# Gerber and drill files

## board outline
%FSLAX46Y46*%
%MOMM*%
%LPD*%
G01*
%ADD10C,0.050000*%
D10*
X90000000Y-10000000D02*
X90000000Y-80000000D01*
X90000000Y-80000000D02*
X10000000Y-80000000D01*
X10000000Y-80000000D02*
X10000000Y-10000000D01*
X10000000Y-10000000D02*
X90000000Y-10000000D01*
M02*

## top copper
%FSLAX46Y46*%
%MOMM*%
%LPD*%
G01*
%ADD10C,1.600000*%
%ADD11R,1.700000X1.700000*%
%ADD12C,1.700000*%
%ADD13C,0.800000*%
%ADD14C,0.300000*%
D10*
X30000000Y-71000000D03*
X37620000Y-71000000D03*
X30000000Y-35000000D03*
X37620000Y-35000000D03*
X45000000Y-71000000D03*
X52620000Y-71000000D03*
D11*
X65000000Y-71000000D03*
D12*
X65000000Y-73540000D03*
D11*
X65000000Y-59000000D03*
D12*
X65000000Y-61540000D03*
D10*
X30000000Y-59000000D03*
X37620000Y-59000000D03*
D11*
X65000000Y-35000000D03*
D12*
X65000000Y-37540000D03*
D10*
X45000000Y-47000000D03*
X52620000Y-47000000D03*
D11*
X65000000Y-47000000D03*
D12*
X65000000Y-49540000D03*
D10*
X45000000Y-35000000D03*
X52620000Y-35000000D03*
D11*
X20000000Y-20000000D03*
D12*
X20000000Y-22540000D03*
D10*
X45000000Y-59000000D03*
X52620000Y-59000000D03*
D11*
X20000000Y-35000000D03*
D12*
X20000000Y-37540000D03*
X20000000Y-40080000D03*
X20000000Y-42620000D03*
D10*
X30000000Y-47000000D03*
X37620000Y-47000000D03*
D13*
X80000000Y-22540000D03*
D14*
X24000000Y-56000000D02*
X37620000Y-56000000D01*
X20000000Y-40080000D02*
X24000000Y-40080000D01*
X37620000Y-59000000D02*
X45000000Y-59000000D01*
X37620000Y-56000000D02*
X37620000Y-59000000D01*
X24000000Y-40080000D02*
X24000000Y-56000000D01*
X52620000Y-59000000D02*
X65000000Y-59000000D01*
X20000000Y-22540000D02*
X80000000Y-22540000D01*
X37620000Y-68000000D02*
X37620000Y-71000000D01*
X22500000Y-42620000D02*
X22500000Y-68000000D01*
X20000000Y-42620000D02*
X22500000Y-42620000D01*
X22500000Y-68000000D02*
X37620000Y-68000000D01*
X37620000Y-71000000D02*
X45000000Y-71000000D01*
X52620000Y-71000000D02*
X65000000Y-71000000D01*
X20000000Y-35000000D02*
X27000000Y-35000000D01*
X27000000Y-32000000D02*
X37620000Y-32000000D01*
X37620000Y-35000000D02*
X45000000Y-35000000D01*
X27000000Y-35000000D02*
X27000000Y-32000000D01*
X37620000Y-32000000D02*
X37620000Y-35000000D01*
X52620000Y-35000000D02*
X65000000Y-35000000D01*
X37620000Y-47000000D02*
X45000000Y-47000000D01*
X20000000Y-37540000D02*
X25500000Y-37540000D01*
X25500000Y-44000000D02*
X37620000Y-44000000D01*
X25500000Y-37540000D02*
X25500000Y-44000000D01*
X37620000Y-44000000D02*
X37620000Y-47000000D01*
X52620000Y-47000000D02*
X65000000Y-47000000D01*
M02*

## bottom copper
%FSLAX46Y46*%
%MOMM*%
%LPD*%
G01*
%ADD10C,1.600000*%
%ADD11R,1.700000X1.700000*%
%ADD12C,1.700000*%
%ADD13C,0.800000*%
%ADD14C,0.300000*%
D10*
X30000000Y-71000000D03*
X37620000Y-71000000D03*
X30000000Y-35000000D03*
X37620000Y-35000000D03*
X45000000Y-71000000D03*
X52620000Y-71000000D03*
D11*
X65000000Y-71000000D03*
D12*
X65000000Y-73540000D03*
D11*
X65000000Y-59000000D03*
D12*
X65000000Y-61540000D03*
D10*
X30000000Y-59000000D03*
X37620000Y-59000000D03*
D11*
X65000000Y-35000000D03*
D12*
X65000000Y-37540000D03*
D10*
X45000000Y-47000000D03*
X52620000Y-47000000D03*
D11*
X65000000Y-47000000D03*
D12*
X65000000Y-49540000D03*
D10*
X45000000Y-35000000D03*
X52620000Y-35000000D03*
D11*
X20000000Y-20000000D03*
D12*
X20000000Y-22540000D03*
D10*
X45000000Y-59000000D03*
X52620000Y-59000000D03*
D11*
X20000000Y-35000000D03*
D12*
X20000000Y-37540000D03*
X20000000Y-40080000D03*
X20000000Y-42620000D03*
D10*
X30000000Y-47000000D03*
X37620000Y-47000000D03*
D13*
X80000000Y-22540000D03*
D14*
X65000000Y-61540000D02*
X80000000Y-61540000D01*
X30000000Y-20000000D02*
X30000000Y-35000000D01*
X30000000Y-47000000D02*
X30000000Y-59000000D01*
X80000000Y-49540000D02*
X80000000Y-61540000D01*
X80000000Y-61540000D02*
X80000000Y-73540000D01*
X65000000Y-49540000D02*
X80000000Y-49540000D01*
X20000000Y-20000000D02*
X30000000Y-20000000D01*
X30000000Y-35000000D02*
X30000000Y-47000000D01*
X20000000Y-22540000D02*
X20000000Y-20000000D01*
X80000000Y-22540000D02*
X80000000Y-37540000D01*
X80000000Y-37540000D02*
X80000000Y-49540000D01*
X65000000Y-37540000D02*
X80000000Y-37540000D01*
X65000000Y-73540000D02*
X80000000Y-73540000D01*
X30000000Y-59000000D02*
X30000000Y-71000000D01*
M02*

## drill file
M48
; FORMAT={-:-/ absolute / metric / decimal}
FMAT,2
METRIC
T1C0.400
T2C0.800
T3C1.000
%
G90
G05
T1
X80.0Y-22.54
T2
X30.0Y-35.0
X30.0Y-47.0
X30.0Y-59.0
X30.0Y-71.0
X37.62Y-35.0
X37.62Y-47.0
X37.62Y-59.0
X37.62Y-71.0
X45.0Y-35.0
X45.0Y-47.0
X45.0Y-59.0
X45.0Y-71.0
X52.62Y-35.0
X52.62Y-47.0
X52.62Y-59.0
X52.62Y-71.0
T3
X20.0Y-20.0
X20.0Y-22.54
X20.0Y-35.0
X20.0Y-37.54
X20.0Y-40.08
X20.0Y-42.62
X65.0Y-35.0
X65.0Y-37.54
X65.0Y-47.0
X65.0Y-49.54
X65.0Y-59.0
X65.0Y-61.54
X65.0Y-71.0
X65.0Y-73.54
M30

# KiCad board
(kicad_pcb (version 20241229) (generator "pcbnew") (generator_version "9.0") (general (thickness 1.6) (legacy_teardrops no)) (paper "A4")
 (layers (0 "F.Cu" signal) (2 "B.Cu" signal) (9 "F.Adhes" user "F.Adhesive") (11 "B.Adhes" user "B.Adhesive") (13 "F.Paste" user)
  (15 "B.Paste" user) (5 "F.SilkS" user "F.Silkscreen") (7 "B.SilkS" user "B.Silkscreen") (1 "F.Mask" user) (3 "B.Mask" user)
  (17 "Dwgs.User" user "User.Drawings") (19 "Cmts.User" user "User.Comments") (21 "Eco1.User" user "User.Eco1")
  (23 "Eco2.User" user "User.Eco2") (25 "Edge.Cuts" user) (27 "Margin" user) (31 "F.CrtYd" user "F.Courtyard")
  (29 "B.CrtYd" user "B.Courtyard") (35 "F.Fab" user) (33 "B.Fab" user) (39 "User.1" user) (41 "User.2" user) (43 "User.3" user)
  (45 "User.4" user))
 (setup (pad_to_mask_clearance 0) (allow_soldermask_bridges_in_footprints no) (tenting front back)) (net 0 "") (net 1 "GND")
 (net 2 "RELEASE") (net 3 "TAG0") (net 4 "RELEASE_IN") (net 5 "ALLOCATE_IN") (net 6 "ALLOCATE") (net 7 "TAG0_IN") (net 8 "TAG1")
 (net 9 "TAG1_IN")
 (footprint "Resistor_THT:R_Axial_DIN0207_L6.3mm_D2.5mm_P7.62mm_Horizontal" (layer "F.Cu") (at 30 71)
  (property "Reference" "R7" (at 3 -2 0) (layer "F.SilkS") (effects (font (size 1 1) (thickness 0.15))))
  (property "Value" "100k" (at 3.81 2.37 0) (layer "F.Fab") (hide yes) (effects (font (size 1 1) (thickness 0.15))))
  (pad "1" thru_hole circle (at 0 0) (size 1.6 1.6) (drill 0.8) (layers "*.Cu" "*.Mask") (remove_unused_layers no) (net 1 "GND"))
  (pad "2" thru_hole circle (at 7.62 0) (size 1.6 1.6) (drill 0.8) (layers "*.Cu" "*.Mask") (remove_unused_layers no) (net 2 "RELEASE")))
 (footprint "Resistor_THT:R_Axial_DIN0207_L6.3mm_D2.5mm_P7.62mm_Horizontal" (layer "F.Cu") (at 30 35)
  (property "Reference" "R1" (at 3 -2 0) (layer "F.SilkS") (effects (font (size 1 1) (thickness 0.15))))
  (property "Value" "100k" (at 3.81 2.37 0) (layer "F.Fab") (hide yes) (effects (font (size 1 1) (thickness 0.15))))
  (pad "1" thru_hole circle (at 0 0) (size 1.6 1.6) (drill 0.8) (layers "*.Cu" "*.Mask") (remove_unused_layers no) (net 1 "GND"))
  (pad "2" thru_hole circle (at 7.62 0) (size 1.6 1.6) (drill 0.8) (layers "*.Cu" "*.Mask") (remove_unused_layers no) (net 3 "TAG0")))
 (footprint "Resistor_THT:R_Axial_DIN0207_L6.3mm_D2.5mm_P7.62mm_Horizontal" (layer "F.Cu") (at 45 71)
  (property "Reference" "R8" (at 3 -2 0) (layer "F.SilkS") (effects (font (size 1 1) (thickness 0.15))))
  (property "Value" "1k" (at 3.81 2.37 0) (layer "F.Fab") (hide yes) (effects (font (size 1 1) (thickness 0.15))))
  (pad "1" thru_hole circle (at 0 0) (size 1.6 1.6) (drill 0.8) (layers "*.Cu" "*.Mask") (remove_unused_layers no) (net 2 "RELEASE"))
  (pad "2" thru_hole circle (at 7.62 0) (size 1.6 1.6) (drill 0.8) (layers "*.Cu" "*.Mask") (remove_unused_layers no) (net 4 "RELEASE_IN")))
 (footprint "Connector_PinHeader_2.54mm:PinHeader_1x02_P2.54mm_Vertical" (layer "F.Cu") (at 65 71)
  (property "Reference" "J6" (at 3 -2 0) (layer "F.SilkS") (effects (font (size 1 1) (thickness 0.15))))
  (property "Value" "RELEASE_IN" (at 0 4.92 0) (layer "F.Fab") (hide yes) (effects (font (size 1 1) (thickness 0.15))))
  (pad "1" thru_hole rect (at 0 0) (size 1.7 1.7) (drill 1) (layers "*.Cu" "*.Mask") (remove_unused_layers no) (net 4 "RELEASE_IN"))
  (pad "2" thru_hole circle (at 0 2.54) (size 1.7 1.7) (drill 1) (layers "*.Cu" "*.Mask") (remove_unused_layers no) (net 1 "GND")))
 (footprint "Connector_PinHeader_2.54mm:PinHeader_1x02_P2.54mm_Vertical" (layer "F.Cu") (at 65 59)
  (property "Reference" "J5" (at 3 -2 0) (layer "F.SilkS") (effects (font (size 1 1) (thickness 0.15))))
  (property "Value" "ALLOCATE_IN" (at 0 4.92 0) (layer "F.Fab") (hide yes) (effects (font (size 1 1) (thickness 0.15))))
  (pad "1" thru_hole rect (at 0 0) (size 1.7 1.7) (drill 1) (layers "*.Cu" "*.Mask") (remove_unused_layers no) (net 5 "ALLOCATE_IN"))
  (pad "2" thru_hole circle (at 0 2.54) (size 1.7 1.7) (drill 1) (layers "*.Cu" "*.Mask") (remove_unused_layers no) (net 1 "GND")))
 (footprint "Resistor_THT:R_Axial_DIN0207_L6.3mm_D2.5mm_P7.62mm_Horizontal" (layer "F.Cu") (at 30 59)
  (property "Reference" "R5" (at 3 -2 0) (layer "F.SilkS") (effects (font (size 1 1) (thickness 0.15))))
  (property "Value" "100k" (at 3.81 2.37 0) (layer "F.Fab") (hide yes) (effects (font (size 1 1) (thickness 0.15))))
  (pad "1" thru_hole circle (at 0 0) (size 1.6 1.6) (drill 0.8) (layers "*.Cu" "*.Mask") (remove_unused_layers no) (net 1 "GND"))
  (pad "2" thru_hole circle (at 7.62 0) (size 1.6 1.6) (drill 0.8) (layers "*.Cu" "*.Mask") (remove_unused_layers no) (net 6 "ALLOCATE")))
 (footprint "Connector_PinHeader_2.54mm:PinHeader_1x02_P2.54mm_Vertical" (layer "F.Cu") (at 65 35)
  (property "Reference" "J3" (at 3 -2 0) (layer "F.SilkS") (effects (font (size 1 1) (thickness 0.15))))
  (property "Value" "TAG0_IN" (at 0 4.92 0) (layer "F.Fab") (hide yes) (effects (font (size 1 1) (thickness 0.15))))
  (pad "1" thru_hole rect (at 0 0) (size 1.7 1.7) (drill 1) (layers "*.Cu" "*.Mask") (remove_unused_layers no) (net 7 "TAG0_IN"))
  (pad "2" thru_hole circle (at 0 2.54) (size 1.7 1.7) (drill 1) (layers "*.Cu" "*.Mask") (remove_unused_layers no) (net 1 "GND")))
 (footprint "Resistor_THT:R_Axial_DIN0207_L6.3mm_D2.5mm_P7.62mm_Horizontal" (layer "F.Cu") (at 45 47)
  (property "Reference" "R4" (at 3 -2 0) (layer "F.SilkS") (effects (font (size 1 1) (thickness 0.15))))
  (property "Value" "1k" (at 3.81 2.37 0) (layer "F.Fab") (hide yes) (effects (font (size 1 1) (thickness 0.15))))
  (pad "1" thru_hole circle (at 0 0) (size 1.6 1.6) (drill 0.8) (layers "*.Cu" "*.Mask") (remove_unused_layers no) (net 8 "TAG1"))
  (pad "2" thru_hole circle (at 7.62 0) (size 1.6 1.6) (drill 0.8) (layers "*.Cu" "*.Mask") (remove_unused_layers no) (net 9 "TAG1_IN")))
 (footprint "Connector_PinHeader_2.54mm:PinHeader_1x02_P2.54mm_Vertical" (layer "F.Cu") (at 65 47)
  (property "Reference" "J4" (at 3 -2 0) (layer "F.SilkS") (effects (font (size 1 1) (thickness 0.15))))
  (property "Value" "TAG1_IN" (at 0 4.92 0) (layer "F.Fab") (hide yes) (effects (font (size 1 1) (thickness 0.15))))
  (pad "1" thru_hole rect (at 0 0) (size 1.7 1.7) (drill 1) (layers "*.Cu" "*.Mask") (remove_unused_layers no) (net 9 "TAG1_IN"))
  (pad "2" thru_hole circle (at 0 2.54) (size 1.7 1.7) (drill 1) (layers "*.Cu" "*.Mask") (remove_unused_layers no) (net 1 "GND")))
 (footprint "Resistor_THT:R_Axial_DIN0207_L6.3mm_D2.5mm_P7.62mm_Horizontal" (layer "F.Cu") (at 45 35)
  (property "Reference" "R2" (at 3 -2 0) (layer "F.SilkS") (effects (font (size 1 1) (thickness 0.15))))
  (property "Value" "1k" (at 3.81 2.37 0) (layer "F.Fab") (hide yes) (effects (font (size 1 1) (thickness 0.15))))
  (pad "1" thru_hole circle (at 0 0) (size 1.6 1.6) (drill 0.8) (layers "*.Cu" "*.Mask") (remove_unused_layers no) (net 3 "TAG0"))
  (pad "2" thru_hole circle (at 7.62 0) (size 1.6 1.6) (drill 0.8) (layers "*.Cu" "*.Mask") (remove_unused_layers no) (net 7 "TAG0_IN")))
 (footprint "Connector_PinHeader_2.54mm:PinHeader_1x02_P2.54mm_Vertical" (layer "F.Cu") (at 20 20)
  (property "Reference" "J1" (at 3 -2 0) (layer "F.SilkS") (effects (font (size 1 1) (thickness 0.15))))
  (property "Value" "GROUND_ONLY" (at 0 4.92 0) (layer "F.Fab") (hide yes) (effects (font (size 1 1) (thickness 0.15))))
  (pad "1" thru_hole rect (at 0 0) (size 1.7 1.7) (drill 1) (layers "*.Cu" "*.Mask") (remove_unused_layers no) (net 1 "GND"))
  (pad "2" thru_hole circle (at 0 2.54) (size 1.7 1.7) (drill 1) (layers "*.Cu" "*.Mask") (remove_unused_layers no) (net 1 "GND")))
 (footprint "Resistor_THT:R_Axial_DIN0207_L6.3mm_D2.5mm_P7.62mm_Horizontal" (layer "F.Cu") (at 45 59)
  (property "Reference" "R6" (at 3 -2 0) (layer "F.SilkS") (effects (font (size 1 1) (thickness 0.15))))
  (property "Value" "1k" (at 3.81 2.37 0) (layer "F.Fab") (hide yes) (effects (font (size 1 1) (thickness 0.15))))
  (pad "1" thru_hole circle (at 0 0) (size 1.6 1.6) (drill 0.8) (layers "*.Cu" "*.Mask") (remove_unused_layers no) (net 6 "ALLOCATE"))
  (pad "2" thru_hole circle (at 7.62 0) (size 1.6 1.6) (drill 0.8) (layers "*.Cu" "*.Mask") (remove_unused_layers no) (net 5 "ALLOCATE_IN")))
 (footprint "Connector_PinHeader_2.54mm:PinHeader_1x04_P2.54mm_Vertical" (layer "F.Cu") (at 20 35)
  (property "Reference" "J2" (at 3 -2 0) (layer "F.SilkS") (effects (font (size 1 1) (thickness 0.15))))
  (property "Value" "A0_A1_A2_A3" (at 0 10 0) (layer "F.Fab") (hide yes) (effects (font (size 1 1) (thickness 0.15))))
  (pad "1" thru_hole rect (at 0 0) (size 1.7 1.7) (drill 1) (layers "*.Cu" "*.Mask") (remove_unused_layers no) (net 3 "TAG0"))
  (pad "2" thru_hole circle (at 0 2.54) (size 1.7 1.7) (drill 1) (layers "*.Cu" "*.Mask") (remove_unused_layers no) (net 8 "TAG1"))
  (pad "3" thru_hole circle (at 0 5.08) (size 1.7 1.7) (drill 1) (layers "*.Cu" "*.Mask") (remove_unused_layers no) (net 6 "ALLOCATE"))
  (pad "4" thru_hole circle (at 0 7.62) (size 1.7 1.7) (drill 1) (layers "*.Cu" "*.Mask") (remove_unused_layers no) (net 2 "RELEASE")))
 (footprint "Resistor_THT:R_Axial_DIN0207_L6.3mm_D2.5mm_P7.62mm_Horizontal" (layer "F.Cu") (at 30 47)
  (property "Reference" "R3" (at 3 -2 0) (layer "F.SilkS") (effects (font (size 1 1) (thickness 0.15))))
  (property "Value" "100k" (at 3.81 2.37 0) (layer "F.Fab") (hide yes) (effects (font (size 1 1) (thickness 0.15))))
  (pad "1" thru_hole circle (at 0 0) (size 1.6 1.6) (drill 0.8) (layers "*.Cu" "*.Mask") (remove_unused_layers no) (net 1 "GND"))
  (pad "2" thru_hole circle (at 7.62 0) (size 1.6 1.6) (drill 0.8) (layers "*.Cu" "*.Mask") (remove_unused_layers no) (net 8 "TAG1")))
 (gr_line (start 90 10) (end 90 80) (stroke (width 0.05) (type default)) (layer "Edge.Cuts"))
 (gr_line (start 90 80) (end 10 80) (stroke (width 0.05) (type default)) (layer "Edge.Cuts"))
 (gr_line (start 10 80) (end 10 10) (stroke (width 0.05) (type default)) (layer "Edge.Cuts"))
 (gr_line (start 10 10) (end 90 10) (stroke (width 0.05) (type default)) (layer "Edge.Cuts"))
 (segment (start 24 56) (end 37.62 56) (width 0.3) (layer "F.Cu") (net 6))
 (segment (start 20 40.08) (end 24 40.08) (width 0.3) (layer "F.Cu") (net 6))
 (segment (start 37.62 59) (end 45 59) (width 0.3) (layer "F.Cu") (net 6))
 (segment (start 37.62 56) (end 37.62 59) (width 0.3) (layer "F.Cu") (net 6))
 (segment (start 24 40.08) (end 24 56) (width 0.3) (layer "F.Cu") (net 6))
 (segment (start 52.62 59) (end 65 59) (width 0.3) (layer "F.Cu") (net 5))
 (segment (start 20 22.54) (end 80 22.54) (width 0.3) (layer "F.Cu") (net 1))
 (via (at 80 22.54) (size 0.8) (drill 0.4) (layers "F.Cu" "B.Cu") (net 1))
 (segment (start 65 61.54) (end 80 61.54) (width 0.3) (layer "B.Cu") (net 1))
 (segment (start 30 20) (end 30 35) (width 0.3) (layer "B.Cu") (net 1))
 (segment (start 30 47) (end 30 59) (width 0.3) (layer "B.Cu") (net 1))
 (segment (start 80 49.54) (end 80 61.54) (width 0.3) (layer "B.Cu") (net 1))
 (segment (start 80 61.54) (end 80 73.54) (width 0.3) (layer "B.Cu") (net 1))
 (segment (start 65 49.54) (end 80 49.54) (width 0.3) (layer "B.Cu") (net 1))
 (segment (start 20 20) (end 30 20) (width 0.3) (layer "B.Cu") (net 1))
 (segment (start 30 35) (end 30 47) (width 0.3) (layer "B.Cu") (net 1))
 (segment (start 20 22.54) (end 20 20) (width 0.3) (layer "B.Cu") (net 1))
 (segment (start 80 22.54) (end 80 37.54) (width 0.3) (layer "B.Cu") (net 1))
 (segment (start 80 37.54) (end 80 49.54) (width 0.3) (layer "B.Cu") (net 1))
 (segment (start 65 37.54) (end 80 37.54) (width 0.3) (layer "B.Cu") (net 1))
 (segment (start 65 73.54) (end 80 73.54) (width 0.3) (layer "B.Cu") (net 1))
 (segment (start 30 59) (end 30 71) (width 0.3) (layer "B.Cu") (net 1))
 (segment (start 37.62 68) (end 37.62 71) (width 0.3) (layer "F.Cu") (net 2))
 (segment (start 22.5 42.62) (end 22.5 68) (width 0.3) (layer "F.Cu") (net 2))
 (segment (start 20 42.62) (end 22.5 42.62) (width 0.3) (layer "F.Cu") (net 2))
 (segment (start 22.5 68) (end 37.62 68) (width 0.3) (layer "F.Cu") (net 2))
 (segment (start 37.62 71) (end 45 71) (width 0.3) (layer "F.Cu") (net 2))
 (segment (start 52.62 71) (end 65 71) (width 0.3) (layer "F.Cu") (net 4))
 (segment (start 20 35) (end 27 35) (width 0.3) (layer "F.Cu") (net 3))
 (segment (start 27 32) (end 37.62 32) (width 0.3) (layer "F.Cu") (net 3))
 (segment (start 37.62 35) (end 45 35) (width 0.3) (layer "F.Cu") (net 3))
 (segment (start 27 35) (end 27 32) (width 0.3) (layer "F.Cu") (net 3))
 (segment (start 37.62 32) (end 37.62 35) (width 0.3) (layer "F.Cu") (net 3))
 (segment (start 52.62 35) (end 65 35) (width 0.3) (layer "F.Cu") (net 7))
 (segment (start 37.62 47) (end 45 47) (width 0.3) (layer "F.Cu") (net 8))
 (segment (start 20 37.54) (end 25.5 37.54) (width 0.3) (layer "F.Cu") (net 8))
 (segment (start 25.5 44) (end 37.62 44) (width 0.3) (layer "F.Cu") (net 8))
 (segment (start 25.5 37.54) (end 25.5 44) (width 0.3) (layer "F.Cu") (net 8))
 (segment (start 37.62 44) (end 37.62 47) (width 0.3) (layer "F.Cu") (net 8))
 (segment (start 52.62 47) (end 65 47) (width 0.3) (layer "F.Cu") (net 9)))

